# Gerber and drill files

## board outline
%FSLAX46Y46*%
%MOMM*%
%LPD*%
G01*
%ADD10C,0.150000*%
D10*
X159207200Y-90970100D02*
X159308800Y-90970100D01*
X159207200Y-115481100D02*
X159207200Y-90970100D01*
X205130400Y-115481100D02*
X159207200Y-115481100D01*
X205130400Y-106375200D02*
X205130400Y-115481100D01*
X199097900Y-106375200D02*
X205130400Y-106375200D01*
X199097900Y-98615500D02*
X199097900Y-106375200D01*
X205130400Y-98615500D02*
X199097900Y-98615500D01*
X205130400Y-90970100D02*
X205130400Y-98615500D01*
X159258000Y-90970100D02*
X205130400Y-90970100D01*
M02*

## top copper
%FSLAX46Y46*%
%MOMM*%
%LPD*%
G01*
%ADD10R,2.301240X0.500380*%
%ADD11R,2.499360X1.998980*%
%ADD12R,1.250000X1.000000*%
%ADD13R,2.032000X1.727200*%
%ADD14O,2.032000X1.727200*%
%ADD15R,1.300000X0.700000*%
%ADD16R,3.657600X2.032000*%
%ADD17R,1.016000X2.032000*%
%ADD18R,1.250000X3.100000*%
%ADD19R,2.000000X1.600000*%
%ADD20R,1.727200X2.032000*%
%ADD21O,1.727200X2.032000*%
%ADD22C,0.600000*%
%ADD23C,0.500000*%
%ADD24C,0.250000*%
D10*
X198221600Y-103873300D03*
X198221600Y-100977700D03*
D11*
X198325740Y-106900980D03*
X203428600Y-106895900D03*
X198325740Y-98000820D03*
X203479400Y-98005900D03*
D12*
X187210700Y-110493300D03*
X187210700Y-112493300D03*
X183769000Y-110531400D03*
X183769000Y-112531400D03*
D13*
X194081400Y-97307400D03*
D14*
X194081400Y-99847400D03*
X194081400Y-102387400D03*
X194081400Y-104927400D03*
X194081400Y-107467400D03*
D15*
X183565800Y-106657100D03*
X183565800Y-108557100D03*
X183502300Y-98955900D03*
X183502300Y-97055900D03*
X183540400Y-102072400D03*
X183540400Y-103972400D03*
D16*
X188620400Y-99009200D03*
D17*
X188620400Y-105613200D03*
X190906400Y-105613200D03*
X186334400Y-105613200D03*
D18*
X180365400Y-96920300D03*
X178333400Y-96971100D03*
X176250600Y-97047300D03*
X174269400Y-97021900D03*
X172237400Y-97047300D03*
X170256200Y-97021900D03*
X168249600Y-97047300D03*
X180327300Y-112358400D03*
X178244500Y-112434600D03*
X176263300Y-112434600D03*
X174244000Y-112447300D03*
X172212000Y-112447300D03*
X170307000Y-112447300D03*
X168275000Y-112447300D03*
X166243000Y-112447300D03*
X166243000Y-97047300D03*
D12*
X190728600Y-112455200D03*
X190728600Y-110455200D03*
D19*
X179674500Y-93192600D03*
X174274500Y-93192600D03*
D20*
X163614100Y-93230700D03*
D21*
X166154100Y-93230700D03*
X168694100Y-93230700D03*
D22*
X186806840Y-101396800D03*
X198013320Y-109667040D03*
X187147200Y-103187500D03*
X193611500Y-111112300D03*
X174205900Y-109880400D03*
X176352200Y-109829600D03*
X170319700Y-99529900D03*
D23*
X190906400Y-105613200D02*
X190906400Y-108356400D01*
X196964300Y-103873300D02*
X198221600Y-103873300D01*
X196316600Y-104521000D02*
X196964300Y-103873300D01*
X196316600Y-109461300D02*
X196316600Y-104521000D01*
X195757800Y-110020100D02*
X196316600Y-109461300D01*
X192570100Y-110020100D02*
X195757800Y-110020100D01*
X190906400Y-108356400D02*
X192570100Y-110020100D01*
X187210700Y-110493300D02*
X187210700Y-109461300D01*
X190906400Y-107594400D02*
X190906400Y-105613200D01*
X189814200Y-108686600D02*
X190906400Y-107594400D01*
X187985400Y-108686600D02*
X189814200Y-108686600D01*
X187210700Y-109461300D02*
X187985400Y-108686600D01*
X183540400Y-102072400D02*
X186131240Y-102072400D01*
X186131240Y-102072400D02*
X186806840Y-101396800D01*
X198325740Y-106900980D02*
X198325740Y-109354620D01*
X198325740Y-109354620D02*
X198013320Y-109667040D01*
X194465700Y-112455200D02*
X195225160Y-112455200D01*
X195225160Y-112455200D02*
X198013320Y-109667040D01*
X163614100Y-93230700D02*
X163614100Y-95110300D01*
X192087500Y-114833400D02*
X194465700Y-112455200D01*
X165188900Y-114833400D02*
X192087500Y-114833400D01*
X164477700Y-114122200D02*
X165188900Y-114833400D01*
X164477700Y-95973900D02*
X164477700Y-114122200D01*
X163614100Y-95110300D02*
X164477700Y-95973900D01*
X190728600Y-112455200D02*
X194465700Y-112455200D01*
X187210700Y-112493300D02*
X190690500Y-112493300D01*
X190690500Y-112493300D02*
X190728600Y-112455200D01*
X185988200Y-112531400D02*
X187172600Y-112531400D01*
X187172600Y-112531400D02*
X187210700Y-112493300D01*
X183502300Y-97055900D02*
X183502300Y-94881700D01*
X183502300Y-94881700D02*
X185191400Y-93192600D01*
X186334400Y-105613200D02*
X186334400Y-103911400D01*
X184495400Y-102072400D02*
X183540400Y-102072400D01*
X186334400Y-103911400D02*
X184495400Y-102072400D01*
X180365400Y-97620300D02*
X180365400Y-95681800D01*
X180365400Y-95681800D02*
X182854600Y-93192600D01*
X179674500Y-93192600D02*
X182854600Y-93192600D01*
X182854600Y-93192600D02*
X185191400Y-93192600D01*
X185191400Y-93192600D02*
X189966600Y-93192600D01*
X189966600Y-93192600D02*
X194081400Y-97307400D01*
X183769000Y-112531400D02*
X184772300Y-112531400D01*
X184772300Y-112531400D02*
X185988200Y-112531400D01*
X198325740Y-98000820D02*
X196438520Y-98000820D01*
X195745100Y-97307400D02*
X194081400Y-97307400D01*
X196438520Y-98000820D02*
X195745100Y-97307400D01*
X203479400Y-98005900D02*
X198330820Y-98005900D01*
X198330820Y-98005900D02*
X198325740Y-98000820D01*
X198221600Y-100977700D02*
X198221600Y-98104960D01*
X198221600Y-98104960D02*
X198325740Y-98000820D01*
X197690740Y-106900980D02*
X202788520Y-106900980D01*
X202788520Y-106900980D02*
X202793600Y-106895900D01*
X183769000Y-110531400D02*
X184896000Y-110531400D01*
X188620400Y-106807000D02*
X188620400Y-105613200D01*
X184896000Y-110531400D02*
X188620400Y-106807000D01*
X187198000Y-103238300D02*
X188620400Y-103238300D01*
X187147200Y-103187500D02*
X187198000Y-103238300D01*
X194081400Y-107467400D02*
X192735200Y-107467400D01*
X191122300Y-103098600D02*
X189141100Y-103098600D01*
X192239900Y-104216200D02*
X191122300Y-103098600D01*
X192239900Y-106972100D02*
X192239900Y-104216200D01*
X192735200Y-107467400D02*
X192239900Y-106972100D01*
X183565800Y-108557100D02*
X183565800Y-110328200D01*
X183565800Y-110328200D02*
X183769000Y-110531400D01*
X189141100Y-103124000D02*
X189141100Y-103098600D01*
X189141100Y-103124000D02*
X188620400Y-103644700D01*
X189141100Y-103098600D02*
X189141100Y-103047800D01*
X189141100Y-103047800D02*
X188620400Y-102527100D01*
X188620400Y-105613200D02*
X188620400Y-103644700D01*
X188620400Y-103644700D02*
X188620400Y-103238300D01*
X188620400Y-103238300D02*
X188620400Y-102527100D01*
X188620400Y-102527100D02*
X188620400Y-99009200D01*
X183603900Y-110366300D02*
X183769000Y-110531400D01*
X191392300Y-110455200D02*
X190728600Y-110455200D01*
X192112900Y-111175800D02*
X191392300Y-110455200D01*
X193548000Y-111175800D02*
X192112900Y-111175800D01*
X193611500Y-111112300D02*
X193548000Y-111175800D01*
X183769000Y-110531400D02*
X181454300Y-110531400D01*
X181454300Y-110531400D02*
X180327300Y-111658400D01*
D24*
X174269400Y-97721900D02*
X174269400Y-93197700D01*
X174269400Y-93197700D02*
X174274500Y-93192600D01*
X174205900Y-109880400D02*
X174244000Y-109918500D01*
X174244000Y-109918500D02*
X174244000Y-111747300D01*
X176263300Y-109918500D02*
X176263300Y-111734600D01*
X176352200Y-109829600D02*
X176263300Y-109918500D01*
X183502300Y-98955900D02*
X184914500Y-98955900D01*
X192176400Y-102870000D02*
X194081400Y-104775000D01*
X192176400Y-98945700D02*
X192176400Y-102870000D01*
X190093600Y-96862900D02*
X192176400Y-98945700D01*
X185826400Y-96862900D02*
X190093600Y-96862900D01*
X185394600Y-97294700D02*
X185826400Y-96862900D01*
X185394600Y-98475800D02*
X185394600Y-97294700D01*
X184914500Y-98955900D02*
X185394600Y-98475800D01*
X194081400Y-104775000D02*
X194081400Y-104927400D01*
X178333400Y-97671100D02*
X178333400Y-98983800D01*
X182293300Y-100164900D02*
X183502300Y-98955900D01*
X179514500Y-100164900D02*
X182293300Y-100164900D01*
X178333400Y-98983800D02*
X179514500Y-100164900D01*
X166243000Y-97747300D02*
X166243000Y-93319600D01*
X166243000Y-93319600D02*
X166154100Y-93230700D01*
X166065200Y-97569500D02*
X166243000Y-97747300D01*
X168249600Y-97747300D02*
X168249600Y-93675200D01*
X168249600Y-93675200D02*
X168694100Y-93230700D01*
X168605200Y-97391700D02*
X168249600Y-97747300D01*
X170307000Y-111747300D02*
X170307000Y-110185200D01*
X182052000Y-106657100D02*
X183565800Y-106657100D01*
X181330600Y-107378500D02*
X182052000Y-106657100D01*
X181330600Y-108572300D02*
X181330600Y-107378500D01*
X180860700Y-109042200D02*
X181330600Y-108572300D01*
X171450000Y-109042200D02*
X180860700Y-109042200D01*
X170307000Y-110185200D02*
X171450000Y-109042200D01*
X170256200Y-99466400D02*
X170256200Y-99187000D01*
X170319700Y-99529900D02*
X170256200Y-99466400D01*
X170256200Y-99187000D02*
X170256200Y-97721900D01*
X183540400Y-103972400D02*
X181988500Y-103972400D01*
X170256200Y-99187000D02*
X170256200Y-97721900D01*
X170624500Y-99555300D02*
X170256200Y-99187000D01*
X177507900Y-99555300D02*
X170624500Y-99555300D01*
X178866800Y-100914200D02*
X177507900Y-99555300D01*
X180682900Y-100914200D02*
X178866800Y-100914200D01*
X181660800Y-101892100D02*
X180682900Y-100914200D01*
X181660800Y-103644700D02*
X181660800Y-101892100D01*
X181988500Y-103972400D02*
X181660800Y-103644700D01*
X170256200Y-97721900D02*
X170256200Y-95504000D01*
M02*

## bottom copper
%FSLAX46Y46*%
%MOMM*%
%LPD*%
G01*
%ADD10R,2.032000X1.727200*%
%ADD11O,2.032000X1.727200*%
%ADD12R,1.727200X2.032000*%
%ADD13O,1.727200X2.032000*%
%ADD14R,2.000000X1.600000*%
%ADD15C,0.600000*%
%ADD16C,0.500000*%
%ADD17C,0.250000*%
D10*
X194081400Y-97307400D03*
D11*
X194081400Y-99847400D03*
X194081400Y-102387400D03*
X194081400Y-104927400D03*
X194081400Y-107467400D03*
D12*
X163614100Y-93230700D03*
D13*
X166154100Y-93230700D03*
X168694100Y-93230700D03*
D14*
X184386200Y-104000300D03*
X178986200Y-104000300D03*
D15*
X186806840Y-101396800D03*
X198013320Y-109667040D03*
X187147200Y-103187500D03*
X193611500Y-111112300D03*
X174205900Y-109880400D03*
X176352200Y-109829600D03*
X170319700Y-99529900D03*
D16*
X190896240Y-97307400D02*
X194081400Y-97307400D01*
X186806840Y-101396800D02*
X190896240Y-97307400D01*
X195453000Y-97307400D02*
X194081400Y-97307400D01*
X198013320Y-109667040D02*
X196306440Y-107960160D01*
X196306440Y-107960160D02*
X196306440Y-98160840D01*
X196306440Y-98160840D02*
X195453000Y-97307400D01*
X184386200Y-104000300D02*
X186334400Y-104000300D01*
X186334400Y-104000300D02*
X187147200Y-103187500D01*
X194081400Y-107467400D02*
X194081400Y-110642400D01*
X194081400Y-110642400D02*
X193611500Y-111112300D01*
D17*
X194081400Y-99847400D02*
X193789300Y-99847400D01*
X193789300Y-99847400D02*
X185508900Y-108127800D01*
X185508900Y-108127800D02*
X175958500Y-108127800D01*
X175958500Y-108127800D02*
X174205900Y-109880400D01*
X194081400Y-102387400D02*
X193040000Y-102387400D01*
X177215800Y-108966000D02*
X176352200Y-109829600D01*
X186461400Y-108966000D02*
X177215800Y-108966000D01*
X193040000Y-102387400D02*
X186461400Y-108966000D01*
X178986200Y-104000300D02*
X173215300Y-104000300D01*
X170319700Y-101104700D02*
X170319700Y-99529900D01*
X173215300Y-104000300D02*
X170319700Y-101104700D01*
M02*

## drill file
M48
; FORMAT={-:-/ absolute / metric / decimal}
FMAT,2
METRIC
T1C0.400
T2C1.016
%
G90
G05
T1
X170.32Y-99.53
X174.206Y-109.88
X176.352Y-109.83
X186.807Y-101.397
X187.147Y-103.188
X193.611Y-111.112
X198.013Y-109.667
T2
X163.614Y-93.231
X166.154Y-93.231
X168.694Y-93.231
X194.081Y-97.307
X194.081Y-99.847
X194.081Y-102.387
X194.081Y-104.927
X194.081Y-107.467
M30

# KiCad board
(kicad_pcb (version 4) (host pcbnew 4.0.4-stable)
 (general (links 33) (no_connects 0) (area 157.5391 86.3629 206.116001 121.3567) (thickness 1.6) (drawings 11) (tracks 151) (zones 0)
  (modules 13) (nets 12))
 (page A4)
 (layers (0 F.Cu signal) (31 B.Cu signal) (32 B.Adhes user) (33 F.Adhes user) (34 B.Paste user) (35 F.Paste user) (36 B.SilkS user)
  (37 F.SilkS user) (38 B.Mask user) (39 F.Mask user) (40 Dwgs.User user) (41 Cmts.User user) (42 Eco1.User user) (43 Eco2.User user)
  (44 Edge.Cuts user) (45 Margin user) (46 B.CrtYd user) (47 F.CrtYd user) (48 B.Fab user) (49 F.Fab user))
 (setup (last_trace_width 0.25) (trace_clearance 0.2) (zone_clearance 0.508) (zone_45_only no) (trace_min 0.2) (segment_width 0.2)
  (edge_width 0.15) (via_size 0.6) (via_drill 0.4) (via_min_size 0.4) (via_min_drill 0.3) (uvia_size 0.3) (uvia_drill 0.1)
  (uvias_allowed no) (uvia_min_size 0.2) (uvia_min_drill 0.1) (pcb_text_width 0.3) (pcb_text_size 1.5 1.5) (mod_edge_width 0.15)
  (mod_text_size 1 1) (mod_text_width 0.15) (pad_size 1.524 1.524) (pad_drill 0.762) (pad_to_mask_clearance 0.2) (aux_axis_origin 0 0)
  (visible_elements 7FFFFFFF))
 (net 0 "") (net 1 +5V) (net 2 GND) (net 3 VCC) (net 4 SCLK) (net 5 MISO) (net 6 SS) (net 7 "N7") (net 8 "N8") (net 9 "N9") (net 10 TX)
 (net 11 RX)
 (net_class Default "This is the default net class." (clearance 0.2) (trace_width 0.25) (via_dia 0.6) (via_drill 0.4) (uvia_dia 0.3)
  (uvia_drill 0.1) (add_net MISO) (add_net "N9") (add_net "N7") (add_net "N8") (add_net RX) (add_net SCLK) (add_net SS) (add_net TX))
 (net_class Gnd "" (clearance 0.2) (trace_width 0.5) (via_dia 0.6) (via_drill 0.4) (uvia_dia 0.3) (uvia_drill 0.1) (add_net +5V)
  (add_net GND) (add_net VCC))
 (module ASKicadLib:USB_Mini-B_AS (layer F.Cu) (at 201.676 102.4509 180)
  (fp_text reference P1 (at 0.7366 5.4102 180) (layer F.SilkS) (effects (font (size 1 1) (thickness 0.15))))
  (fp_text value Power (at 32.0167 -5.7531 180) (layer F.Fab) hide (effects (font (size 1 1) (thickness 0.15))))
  (pad 1 smd rect (at 3.4544 -1.4224 180) (size 2.30124 0.50038) (layers F.Cu F.Paste F.Mask) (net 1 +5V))
  (pad 5 smd rect (at 3.4544 1.4732 180) (size 2.30124 0.50038) (layers F.Cu F.Paste F.Mask) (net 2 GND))
  (pad 6 smd rect (at 3.35026 -4.45008 180) (size 2.49936 1.99898) (layers F.Cu F.Paste F.Mask) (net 2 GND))
  (pad 6 smd rect (at -1.7526 -4.445 180) (size 2.49936 1.99898) (layers F.Cu F.Paste F.Mask) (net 2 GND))
  (pad 6 smd rect (at 3.35026 4.45008 180) (size 2.49936 1.99898) (layers F.Cu F.Paste F.Mask) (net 2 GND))
  (pad 6 smd rect (at -1.8034 4.445 180) (size 2.49936 1.99898) (layers F.Cu F.Paste F.Mask) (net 2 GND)))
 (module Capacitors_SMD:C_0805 (layer F.Cu) (at 187.2107 111.4933 270)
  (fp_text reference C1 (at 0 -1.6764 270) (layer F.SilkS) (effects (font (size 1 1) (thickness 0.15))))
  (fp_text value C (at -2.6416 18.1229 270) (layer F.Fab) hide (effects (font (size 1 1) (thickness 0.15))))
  (pad 1 smd rect (at -1 0 270) (size 1 1.25) (layers F.Cu F.Paste F.Mask) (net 1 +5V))
  (pad 2 smd rect (at 1 0 270) (size 1 1.25) (layers F.Cu F.Paste F.Mask) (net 2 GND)))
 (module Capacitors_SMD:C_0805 (layer F.Cu) (at 183.769 111.5314 270)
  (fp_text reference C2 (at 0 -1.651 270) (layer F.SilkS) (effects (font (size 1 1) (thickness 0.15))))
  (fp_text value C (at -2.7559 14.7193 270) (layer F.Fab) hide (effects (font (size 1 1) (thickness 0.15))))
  (pad 1 smd rect (at -1 0 270) (size 1 1.25) (layers F.Cu F.Paste F.Mask) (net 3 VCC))
  (pad 2 smd rect (at 1 0 270) (size 1 1.25) (layers F.Cu F.Paste F.Mask) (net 2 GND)))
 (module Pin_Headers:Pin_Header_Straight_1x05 (layer F.Cu) (at 194.0814 97.3074)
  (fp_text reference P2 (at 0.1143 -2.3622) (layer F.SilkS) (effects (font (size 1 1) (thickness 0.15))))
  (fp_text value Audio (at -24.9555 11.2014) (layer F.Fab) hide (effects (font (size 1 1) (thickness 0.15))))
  (pad 1 thru_hole rect (at 0 0) (size 2.032 1.7272) (drill 1.016) (layers *.Cu *.Mask) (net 2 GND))
  (pad 2 thru_hole oval (at 0 2.54) (size 2.032 1.7272) (drill 1.016) (layers *.Cu *.Mask) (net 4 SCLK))
  (pad 3 thru_hole oval (at 0 5.08) (size 2.032 1.7272) (drill 1.016) (layers *.Cu *.Mask) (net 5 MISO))
  (pad 4 thru_hole oval (at 0 7.62) (size 2.032 1.7272) (drill 1.016) (layers *.Cu *.Mask) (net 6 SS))
  (pad 5 thru_hole oval (at 0 10.16) (size 2.032 1.7272) (drill 1.016) (layers *.Cu *.Mask) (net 3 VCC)))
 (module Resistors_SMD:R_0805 (layer F.Cu) (at 183.5658 107.6071 270)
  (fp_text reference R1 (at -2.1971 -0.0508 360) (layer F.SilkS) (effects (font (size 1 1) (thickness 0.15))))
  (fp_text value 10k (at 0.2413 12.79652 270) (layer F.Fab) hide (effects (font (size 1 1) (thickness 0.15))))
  (pad 1 smd rect (at -0.95 0 270) (size 0.7 1.3) (layers F.Cu F.Paste F.Mask) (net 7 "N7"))
  (pad 2 smd rect (at 0.95 0 270) (size 0.7 1.3) (layers F.Cu F.Paste F.Mask) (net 3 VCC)))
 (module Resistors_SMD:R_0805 (layer F.Cu) (at 183.5023 98.0059 90)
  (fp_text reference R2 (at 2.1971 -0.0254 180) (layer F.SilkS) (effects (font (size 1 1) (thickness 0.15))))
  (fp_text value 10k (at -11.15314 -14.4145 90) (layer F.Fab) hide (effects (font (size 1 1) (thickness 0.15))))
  (pad 1 smd rect (at -0.95 0 90) (size 0.7 1.3) (layers F.Cu F.Paste F.Mask) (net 6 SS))
  (pad 2 smd rect (at 0.95 0 90) (size 0.7 1.3) (layers F.Cu F.Paste F.Mask) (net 2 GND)))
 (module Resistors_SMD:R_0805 (layer F.Cu) (at 183.5404 103.0224 270)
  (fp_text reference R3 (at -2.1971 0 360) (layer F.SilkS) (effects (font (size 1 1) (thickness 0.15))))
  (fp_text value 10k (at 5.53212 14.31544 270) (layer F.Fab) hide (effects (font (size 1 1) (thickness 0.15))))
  (pad 1 smd rect (at -0.95 0 270) (size 0.7 1.3) (layers F.Cu F.Paste F.Mask) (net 2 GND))
  (pad 2 smd rect (at 0.95 0 270) (size 0.7 1.3) (layers F.Cu F.Paste F.Mask) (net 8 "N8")))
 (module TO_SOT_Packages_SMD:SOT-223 (layer F.Cu) (at 188.6204 102.3112)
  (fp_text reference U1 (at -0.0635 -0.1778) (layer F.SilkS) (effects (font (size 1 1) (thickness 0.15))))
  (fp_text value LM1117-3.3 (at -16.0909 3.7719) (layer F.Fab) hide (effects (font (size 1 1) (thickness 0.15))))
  (pad 4 smd rect (at 0 -3.302) (size 3.6576 2.032) (layers F.Cu F.Paste F.Mask) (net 3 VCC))
  (pad 2 smd rect (at 0 3.302) (size 1.016 2.032) (layers F.Cu F.Paste F.Mask) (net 3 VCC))
  (pad 3 smd rect (at 2.286 3.302) (size 1.016 2.032) (layers F.Cu F.Paste F.Mask) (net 1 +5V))
  (pad 1 smd rect (at -2.286 3.302) (size 1.016 2.032) (layers F.Cu F.Paste F.Mask) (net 2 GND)))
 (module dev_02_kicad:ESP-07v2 (layer F.Cu) (at 166.243 111.7473 90)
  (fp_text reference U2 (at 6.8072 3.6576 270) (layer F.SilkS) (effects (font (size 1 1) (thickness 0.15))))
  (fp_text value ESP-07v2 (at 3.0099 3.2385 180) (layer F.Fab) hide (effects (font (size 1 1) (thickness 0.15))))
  (pad 9 smd rect (at 14.127 14.1224 90) (size 3.1 1.25) (drill (offset 0.7 0)) (layers F.Cu F.Paste F.Mask) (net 2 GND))
  (pad 10 smd rect (at 14.0762 12.0904 90) (size 3.1 1.25) (drill (offset 0.7 0)) (layers F.Cu F.Paste F.Mask) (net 6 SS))
  (pad 11 smd rect (at 14 10.0076 90) (size 3.1 1.25) (drill (offset 0.7 0)) (layers F.Cu F.Paste F.Mask))
  (pad 12 smd rect (at 14.0254 8.0264 90) (size 3.1 1.25) (drill (offset 0.7 0)) (layers F.Cu F.Paste F.Mask) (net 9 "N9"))
  (pad 13 smd rect (at 14 5.9944 90) (size 3.1 1.25) (drill (offset 0.7 0)) (layers F.Cu F.Paste F.Mask))
  (pad 14 smd rect (at 14.0254 4.0132 90) (size 3.1 1.25) (drill (offset 0.7 0)) (layers F.Cu F.Paste F.Mask) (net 8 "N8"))
  (pad 15 smd rect (at 14 2.0066 90) (size 3.1 1.25) (drill (offset 0.7 0)) (layers F.Cu F.Paste F.Mask) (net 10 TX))
  (pad 8 smd rect (at 0.0889 14.0843 90) (size 3.1 1.25) (drill (offset -0.7 0)) (layers F.Cu F.Paste F.Mask) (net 3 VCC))
  (pad 7 smd rect (at 0.0127 12.0015 90) (size 3.1 1.25) (drill (offset -0.7 0)) (layers F.Cu F.Paste F.Mask))
  (pad 6 smd rect (at 0.0127 10.0203 90) (size 3.1 1.25) (drill (offset -0.7 0)) (layers F.Cu F.Paste F.Mask) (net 5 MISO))
  (pad 5 smd rect (at 0 8.001 90) (size 3.1 1.25) (drill (offset -0.7 0)) (layers F.Cu F.Paste F.Mask) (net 4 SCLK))
  (pad 4 smd rect (at 0 5.969 90) (size 3.1 1.25) (drill (offset -0.7 0)) (layers F.Cu F.Paste F.Mask))
  (pad 3 smd rect (at 0 4.064 90) (size 3.1 1.25) (drill (offset -0.7 0)) (layers F.Cu F.Paste F.Mask) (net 7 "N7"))
  (pad 2 smd rect (at 0 2.032 90) (size 3.1 1.25) (drill (offset -0.7 0)) (layers F.Cu F.Paste F.Mask))
  (pad 1 smd rect (at 0 0 90) (size 3.1 1.25) (drill (offset -0.7 0)) (layers F.Cu F.Paste F.Mask))
  (pad 16 smd rect (at 14 0 90) (size 3.1 1.25) (drill (offset 0.7 0)) (layers F.Cu F.Paste F.Mask) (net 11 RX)))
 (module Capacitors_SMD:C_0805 (layer F.Cu) (at 190.7286 111.4552 90)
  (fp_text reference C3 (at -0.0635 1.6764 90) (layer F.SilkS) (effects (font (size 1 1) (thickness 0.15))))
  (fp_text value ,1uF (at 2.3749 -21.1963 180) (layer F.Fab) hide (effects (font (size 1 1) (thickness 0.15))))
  (pad 1 smd rect (at -1 0 90) (size 1 1.25) (layers F.Cu F.Paste F.Mask) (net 2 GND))
  (pad 2 smd rect (at 1 0 90) (size 1 1.25) (layers F.Cu F.Paste F.Mask) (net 3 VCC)))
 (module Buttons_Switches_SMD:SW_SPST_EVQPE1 (layer F.Cu) (at 176.9745 93.1926)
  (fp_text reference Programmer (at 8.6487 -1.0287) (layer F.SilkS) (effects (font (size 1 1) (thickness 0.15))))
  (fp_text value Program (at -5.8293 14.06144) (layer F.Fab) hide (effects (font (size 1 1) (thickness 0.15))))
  (pad 2 smd rect (at 2.7 0) (size 2 1.6) (layers F.Cu F.Paste F.Mask) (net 2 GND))
  (pad 1 smd rect (at -2.7 0) (size 2 1.6) (layers F.Cu F.Paste F.Mask) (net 9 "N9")))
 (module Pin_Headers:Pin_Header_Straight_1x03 (layer F.Cu) (at 163.6141 93.2307 90)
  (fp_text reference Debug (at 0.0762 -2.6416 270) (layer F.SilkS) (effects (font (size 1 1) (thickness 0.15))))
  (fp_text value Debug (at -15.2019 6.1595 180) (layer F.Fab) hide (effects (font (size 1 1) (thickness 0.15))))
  (pad 1 thru_hole rect (at 0 0 90) (size 2.032 1.7272) (drill 1.016) (layers *.Cu *.Mask) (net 2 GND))
  (pad 2 thru_hole oval (at 0 2.54 90) (size 2.032 1.7272) (drill 1.016) (layers *.Cu *.Mask) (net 11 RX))
  (pad 3 thru_hole oval (at 0 5.08 90) (size 2.032 1.7272) (drill 1.016) (layers *.Cu *.Mask) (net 10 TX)))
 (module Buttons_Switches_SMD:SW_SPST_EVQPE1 (layer B.Cu) (at 181.6862 104.0003)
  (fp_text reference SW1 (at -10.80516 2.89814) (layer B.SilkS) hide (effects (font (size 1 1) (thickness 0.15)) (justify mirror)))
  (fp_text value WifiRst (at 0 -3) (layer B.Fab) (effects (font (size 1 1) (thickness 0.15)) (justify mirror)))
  (pad 2 smd rect (at 2.7 0) (size 2 1.6) (layers B.Cu B.Paste B.Mask) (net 3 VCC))
  (pad 1 smd rect (at -2.7 0) (size 2 1.6) (layers B.Cu B.Paste B.Mask) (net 8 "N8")))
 (gr_line (start 159.2072 90.9701) (end 159.3088 90.9701) (angle 90) (layer Edge.Cuts) (width 0.15))
 (gr_line (start 159.2072 115.4811) (end 159.2072 90.9701) (angle 90) (layer Edge.Cuts) (width 0.15))
 (gr_line (start 205.1304 115.4811) (end 159.2072 115.4811) (angle 90) (layer Edge.Cuts) (width 0.15))
 (gr_line (start 205.1304 106.3752) (end 205.1304 115.4811) (angle 90) (layer Edge.Cuts) (width 0.15))
 (gr_line (start 199.0979 106.3752) (end 205.1304 106.3752) (angle 90) (layer Edge.Cuts) (width 0.15))
 (gr_line (start 199.0979 98.6155) (end 199.0979 106.3752) (angle 90) (layer Edge.Cuts) (width 0.15))
 (gr_line (start 205.1304 98.6155) (end 199.0979 98.6155) (angle 90) (layer Edge.Cuts) (width 0.15))
 (gr_line (start 205.1304 90.9701) (end 205.1304 98.6155) (angle 90) (layer Edge.Cuts) (width 0.15))
 (gr_line (start 159.258 90.9701) (end 205.1304 90.9701) (angle 90) (layer Edge.Cuts) (width 0.15))
 (segment (start 190.9064 105.6132) (end 190.9064 108.3564) (width 0.5) (layer F.Cu) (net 1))
 (segment (start 196.9643 103.8733) (end 198.2216 103.8733) (width 0.5) (layer F.Cu) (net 1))
 (segment (start 196.3166 104.521) (end 196.9643 103.8733) (width 0.5) (layer F.Cu) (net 1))
 (segment (start 196.3166 109.4613) (end 196.3166 104.521) (width 0.5) (layer F.Cu) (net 1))
 (segment (start 195.7578 110.0201) (end 196.3166 109.4613) (width 0.5) (layer F.Cu) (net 1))
 (segment (start 192.5701 110.0201) (end 195.7578 110.0201) (width 0.5) (layer F.Cu) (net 1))
 (segment (start 190.9064 108.3564) (end 192.5701 110.0201) (width 0.5) (layer F.Cu) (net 1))
 (segment (start 187.2107 110.4933) (end 187.2107 109.4613) (width 0.5) (layer F.Cu) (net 1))
 (segment (start 190.9064 107.5944) (end 190.9064 105.6132) (width 0.5) (layer F.Cu) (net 1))
 (segment (start 189.8142 108.6866) (end 190.9064 107.5944) (width 0.5) (layer F.Cu) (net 1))
 (segment (start 187.9854 108.6866) (end 189.8142 108.6866) (width 0.5) (layer F.Cu) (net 1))
 (segment (start 187.2107 109.4613) (end 187.9854 108.6866) (width 0.5) (layer F.Cu) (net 1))
 (segment (start 183.5404 102.0724) (end 186.13124 102.0724) (width 0.5) (layer F.Cu) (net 2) (status 400000))
 (segment (start 190.89624 97.3074) (end 194.0814 97.3074) (width 0.5) (layer B.Cu) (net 2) (status 800000))
 (segment (start 186.80684 101.3968) (end 190.89624 97.3074) (width 0.5) (layer B.Cu) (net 2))
 (via (at 186.80684 101.3968) (size 0.6) (drill 0.4) (layers F.Cu B.Cu) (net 2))
 (segment (start 186.13124 102.0724) (end 186.80684 101.3968) (width 0.5) (layer F.Cu) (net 2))
 (segment (start 198.32574 106.90098) (end 198.32574 109.35462) (width 0.5) (layer F.Cu) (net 2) (status 400000))
 (segment (start 198.32574 109.35462) (end 198.01332 109.66704) (width 0.5) (layer F.Cu) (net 2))
 (segment (start 194.4657 112.4552) (end 195.22516 112.4552) (width 0.5) (layer F.Cu) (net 2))
 (segment (start 195.453 97.3074) (end 194.0814 97.3074) (width 0.5) (layer B.Cu) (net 2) (status 800000))
 (via (at 198.01332 109.66704) (size 0.6) (drill 0.4) (layers F.Cu B.Cu) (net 2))
 (segment (start 198.01332 109.66704) (end 196.30644 107.96016) (width 0.5) (layer B.Cu) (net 2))
 (segment (start 196.30644 107.96016) (end 196.30644 98.16084) (width 0.5) (layer B.Cu) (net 2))
 (segment (start 196.30644 98.16084) (end 195.453 97.3074) (width 0.5) (layer B.Cu) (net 2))
 (segment (start 195.22516 112.4552) (end 198.01332 109.66704) (width 0.5) (layer F.Cu) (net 2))
 (segment (start 163.6141 93.2307) (end 163.6141 95.1103) (width 0.5) (layer F.Cu) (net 2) (status 400000))
 (segment (start 192.0875 114.8334) (end 194.4657 112.4552) (width 0.5) (layer F.Cu) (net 2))
 (segment (start 165.1889 114.8334) (end 192.0875 114.8334) (width 0.5) (layer F.Cu) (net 2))
 (segment (start 164.4777 114.1222) (end 165.1889 114.8334) (width 0.5) (layer F.Cu) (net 2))
 (segment (start 164.4777 95.9739) (end 164.4777 114.1222) (width 0.5) (layer F.Cu) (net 2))
 (segment (start 163.6141 95.1103) (end 164.4777 95.9739) (width 0.5) (layer F.Cu) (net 2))
 (segment (start 190.7286 112.4552) (end 194.4657 112.4552) (width 0.5) (layer F.Cu) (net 2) (status 400000))
 (segment (start 187.2107 112.4933) (end 190.6905 112.4933) (width 0.5) (layer F.Cu) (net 2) (status C00000))
 (segment (start 190.6905 112.4933) (end 190.7286 112.4552) (width 0.5) (layer F.Cu) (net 2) (status C00000))
 (segment (start 185.9882 112.5314) (end 187.1726 112.5314) (width 0.5) (layer F.Cu) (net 2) (status 800000))
 (segment (start 187.1726 112.5314) (end 187.2107 112.4933) (width 0.5) (layer F.Cu) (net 2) (status C00000))
 (segment (start 183.5023 97.0559) (end 183.5023 94.8817) (width 0.5) (layer F.Cu) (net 2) (status 400000))
 (segment (start 183.5023 94.8817) (end 185.1914 93.1926) (width 0.5) (layer F.Cu) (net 2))
 (segment (start 186.3344 105.6132) (end 186.3344 103.9114) (width 0.5) (layer F.Cu) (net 2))
 (segment (start 184.4954 102.0724) (end 183.5404 102.0724) (width 0.5) (layer F.Cu) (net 2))
 (segment (start 186.3344 103.9114) (end 184.4954 102.0724) (width 0.5) (layer F.Cu) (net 2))
 (segment (start 180.3654 97.6203) (end 180.3654 95.6818) (width 0.5) (layer F.Cu) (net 2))
 (segment (start 180.3654 95.6818) (end 182.8546 93.1926) (width 0.5) (layer F.Cu) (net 2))
 (segment (start 179.6745 93.1926) (end 182.8546 93.1926) (width 0.5) (layer F.Cu) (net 2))
 (segment (start 182.8546 93.1926) (end 185.1914 93.1926) (width 0.5) (layer F.Cu) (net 2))
 (segment (start 185.1914 93.1926) (end 189.9666 93.1926) (width 0.5) (layer F.Cu) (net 2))
 (segment (start 189.9666 93.1926) (end 194.0814 97.3074) (width 0.5) (layer F.Cu) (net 2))
 (segment (start 183.769 112.5314) (end 184.7723 112.5314) (width 0.5) (layer F.Cu) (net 2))
 (segment (start 184.7723 112.5314) (end 185.9882 112.5314) (width 0.5) (layer F.Cu) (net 2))
 (segment (start 198.32574 98.00082) (end 196.43852 98.00082) (width 0.5) (layer F.Cu) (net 2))
 (segment (start 195.7451 97.3074) (end 194.0814 97.3074) (width 0.5) (layer F.Cu) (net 2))
 (segment (start 196.43852 98.00082) (end 195.7451 97.3074) (width 0.5) (layer F.Cu) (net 2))
 (segment (start 203.4794 98.0059) (end 198.33082 98.0059) (width 0.5) (layer F.Cu) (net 2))
 (segment (start 198.33082 98.0059) (end 198.32574 98.00082) (width 0.5) (layer F.Cu) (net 2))
 (segment (start 198.2216 100.9777) (end 198.2216 98.10496) (width 0.5) (layer F.Cu) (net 2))
 (segment (start 198.2216 98.10496) (end 198.32574 98.00082) (width 0.5) (layer F.Cu) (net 2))
 (segment (start 197.69074 106.90098) (end 202.78852 106.90098) (width 0.5) (layer F.Cu) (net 2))
 (segment (start 202.78852 106.90098) (end 202.7936 106.8959) (width 0.5) (layer F.Cu) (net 2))
 (segment (start 183.769 110.5314) (end 184.896 110.5314) (width 0.5) (layer F.Cu) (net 3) (status 400000))
 (segment (start 188.6204 106.807) (end 188.6204 105.6132) (width 0.5) (layer F.Cu) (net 3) (status 800000))
 (segment (start 184.896 110.5314) (end 188.6204 106.807) (width 0.5) (layer F.Cu) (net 3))
 (segment (start 184.3862 104.0003) (end 186.3344 104.0003) (width 0.5) (layer B.Cu) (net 3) (status 400000))
 (segment (start 187.198 103.2383) (end 188.6204 103.2383) (width 0.5) (layer F.Cu) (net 3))
 (segment (start 187.1472 103.1875) (end 187.198 103.2383) (width 0.5) (layer F.Cu) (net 3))
 (via (at 187.1472 103.1875) (size 0.6) (drill 0.4) (layers F.Cu B.Cu) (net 3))
 (segment (start 186.3344 104.0003) (end 187.1472 103.1875) (width 0.5) (layer B.Cu) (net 3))
 (segment (start 194.0814 107.4674) (end 192.7352 107.4674) (width 0.5) (layer F.Cu) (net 3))
 (segment (start 191.1223 103.0986) (end 189.1411 103.0986) (width 0.5) (layer F.Cu) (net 3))
 (segment (start 192.2399 104.2162) (end 191.1223 103.0986) (width 0.5) (layer F.Cu) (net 3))
 (segment (start 192.2399 106.9721) (end 192.2399 104.2162) (width 0.5) (layer F.Cu) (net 3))
 (segment (start 192.7352 107.4674) (end 192.2399 106.9721) (width 0.5) (layer F.Cu) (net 3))
 (segment (start 183.5658 108.5571) (end 183.5658 110.3282) (width 0.5) (layer F.Cu) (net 3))
 (segment (start 183.5658 110.3282) (end 183.769 110.5314) (width 0.5) (layer F.Cu) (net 3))
 (segment (start 189.1411 103.124) (end 189.1411 103.0986) (width 0.5) (layer F.Cu) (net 3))
 (segment (start 189.1411 103.124) (end 188.6204 103.6447) (width 0.5) (layer F.Cu) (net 3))
 (segment (start 189.1411 103.0986) (end 189.1411 103.0478) (width 0.5) (layer F.Cu) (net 3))
 (segment (start 189.1411 103.0478) (end 188.6204 102.5271) (width 0.5) (layer F.Cu) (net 3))
 (segment (start 188.6204 105.6132) (end 188.6204 103.6447) (width 0.5) (layer F.Cu) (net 3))
 (segment (start 188.6204 103.6447) (end 188.6204 103.2383) (width 0.5) (layer F.Cu) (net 3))
 (segment (start 188.6204 103.2383) (end 188.6204 102.5271) (width 0.5) (layer F.Cu) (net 3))
 (segment (start 188.6204 102.5271) (end 188.6204 99.0092) (width 0.5) (layer F.Cu) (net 3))
 (segment (start 183.6039 110.3663) (end 183.769 110.5314) (width 0.5) (layer F.Cu) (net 3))
 (segment (start 194.0814 107.4674) (end 194.0814 110.6424) (width 0.5) (layer B.Cu) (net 3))
 (segment (start 191.3923 110.4552) (end 190.7286 110.4552) (width 0.5) (layer F.Cu) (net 3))
 (segment (start 192.1129 111.1758) (end 191.3923 110.4552) (width 0.5) (layer F.Cu) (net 3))
 (segment (start 193.548 111.1758) (end 192.1129 111.1758) (width 0.5) (layer F.Cu) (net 3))
 (segment (start 193.6115 111.1123) (end 193.548 111.1758) (width 0.5) (layer F.Cu) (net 3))
 (via (at 193.6115 111.1123) (size 0.6) (drill 0.4) (layers F.Cu B.Cu) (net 3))
 (segment (start 194.0814 110.6424) (end 193.6115 111.1123) (width 0.5) (layer B.Cu) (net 3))
 (segment (start 183.769 110.5314) (end 181.4543 110.5314) (width 0.5) (layer F.Cu) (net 3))
 (segment (start 181.4543 110.5314) (end 180.3273 111.6584) (width 0.5) (layer F.Cu) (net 3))
 (segment (start 174.2694 97.7219) (end 174.2694 93.1977) (width 0.25) (layer F.Cu) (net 9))
 (segment (start 174.2694 93.1977) (end 174.2745 93.1926) (width 0.25) (layer F.Cu) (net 9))
 (segment (start 194.0814 99.8474) (end 193.7893 99.8474) (width 0.25) (layer B.Cu) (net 4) (status C00000))
 (segment (start 193.7893 99.8474) (end 185.5089 108.1278) (width 0.25) (layer B.Cu) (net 4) (status 400000))
 (segment (start 185.5089 108.1278) (end 175.9585 108.1278) (width 0.25) (layer B.Cu) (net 4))
 (segment (start 175.9585 108.1278) (end 174.2059 109.8804) (width 0.25) (layer B.Cu) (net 4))
 (via (at 174.2059 109.8804) (size 0.6) (drill 0.4) (layers F.Cu B.Cu) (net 4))
 (segment (start 174.2059 109.8804) (end 174.244 109.9185) (width 0.25) (layer F.Cu) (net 4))
 (segment (start 174.244 109.9185) (end 174.244 111.7473) (width 0.25) (layer F.Cu) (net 4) (status 800000))
 (segment (start 194.0814 102.3874) (end 193.04 102.3874) (width 0.25) (layer B.Cu) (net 5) (status 400000))
 (segment (start 176.2633 109.9185) (end 176.2633 111.7346) (width 0.25) (layer F.Cu) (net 5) (status 800000))
 (segment (start 176.3522 109.8296) (end 176.2633 109.9185) (width 0.25) (layer F.Cu) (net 5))
 (via (at 176.3522 109.8296) (size 0.6) (drill 0.4) (layers F.Cu B.Cu) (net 5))
 (segment (start 177.2158 108.966) (end 176.3522 109.8296) (width 0.25) (layer B.Cu) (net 5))
 (segment (start 186.4614 108.966) (end 177.2158 108.966) (width 0.25) (layer B.Cu) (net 5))
 (segment (start 193.04 102.3874) (end 186.4614 108.966) (width 0.25) (layer B.Cu) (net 5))
 (segment (start 183.5023 98.9559) (end 184.9145 98.9559) (width 0.25) (layer F.Cu) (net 6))
 (segment (start 192.1764 102.87) (end 194.0814 104.775) (width 0.25) (layer F.Cu) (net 6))
 (segment (start 192.1764 98.9457) (end 192.1764 102.87) (width 0.25) (layer F.Cu) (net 6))
 (segment (start 190.0936 96.8629) (end 192.1764 98.9457) (width 0.25) (layer F.Cu) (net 6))
 (segment (start 185.8264 96.8629) (end 190.0936 96.8629) (width 0.25) (layer F.Cu) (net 6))
 (segment (start 185.3946 97.2947) (end 185.8264 96.8629) (width 0.25) (layer F.Cu) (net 6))
 (segment (start 185.3946 98.4758) (end 185.3946 97.2947) (width 0.25) (layer F.Cu) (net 6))
 (segment (start 184.9145 98.9559) (end 185.3946 98.4758) (width 0.25) (layer F.Cu) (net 6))
 (segment (start 194.0814 104.775) (end 194.0814 104.9274) (width 0.25) (layer F.Cu) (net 6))
 (segment (start 178.3334 97.6711) (end 178.3334 98.9838) (width 0.25) (layer F.Cu) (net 6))
 (segment (start 182.2933 100.1649) (end 183.5023 98.9559) (width 0.25) (layer F.Cu) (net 6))
 (segment (start 179.5145 100.1649) (end 182.2933 100.1649) (width 0.25) (layer F.Cu) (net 6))
 (segment (start 178.3334 98.9838) (end 179.5145 100.1649) (width 0.25) (layer F.Cu) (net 6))
 (segment (start 166.243 97.7473) (end 166.243 93.3196) (width 0.25) (layer F.Cu) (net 11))
 (segment (start 166.243 93.3196) (end 166.1541 93.2307) (width 0.25) (layer F.Cu) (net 11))
 (segment (start 166.0652 97.5695) (end 166.243 97.7473) (width 0.25) (layer F.Cu) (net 11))
 (segment (start 168.2496 97.7473) (end 168.2496 93.6752) (width 0.25) (layer F.Cu) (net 10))
 (segment (start 168.2496 93.6752) (end 168.6941 93.2307) (width 0.25) (layer F.Cu) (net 10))
 (segment (start 168.6052 97.3917) (end 168.2496 97.7473) (width 0.25) (layer F.Cu) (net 10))
 (segment (start 170.307 111.7473) (end 170.307 110.1852) (width 0.25) (layer F.Cu) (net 7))
 (segment (start 182.052 106.6571) (end 183.5658 106.6571) (width 0.25) (layer F.Cu) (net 7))
 (segment (start 181.3306 107.3785) (end 182.052 106.6571) (width 0.25) (layer F.Cu) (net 7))
 (segment (start 181.3306 108.5723) (end 181.3306 107.3785) (width 0.25) (layer F.Cu) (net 7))
 (segment (start 180.8607 109.0422) (end 181.3306 108.5723) (width 0.25) (layer F.Cu) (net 7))
 (segment (start 171.45 109.0422) (end 180.8607 109.0422) (width 0.25) (layer F.Cu) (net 7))
 (segment (start 170.307 110.1852) (end 171.45 109.0422) (width 0.25) (layer F.Cu) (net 7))
 (segment (start 178.9862 104.0003) (end 173.2153 104.0003) (width 0.25) (layer B.Cu) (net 8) (status 400000))
 (segment (start 170.2562 99.4664) (end 170.2562 99.187) (width 0.25) (layer F.Cu) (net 8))
 (segment (start 170.3197 99.5299) (end 170.2562 99.4664) (width 0.25) (layer F.Cu) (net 8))
 (via (at 170.3197 99.5299) (size 0.6) (drill 0.4) (layers F.Cu B.Cu) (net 8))
 (segment (start 170.3197 101.1047) (end 170.3197 99.5299) (width 0.25) (layer B.Cu) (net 8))
 (segment (start 173.2153 104.0003) (end 170.3197 101.1047) (width 0.25) (layer B.Cu) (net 8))
 (segment (start 170.2562 99.187) (end 170.2562 97.7219) (width 0.25) (layer F.Cu) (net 8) (status 800000))
 (segment (start 183.5404 103.9724) (end 181.9885 103.9724) (width 0.25) (layer F.Cu) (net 8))
 (segment (start 170.2562 99.187) (end 170.2562 97.7219) (width 0.25) (layer F.Cu) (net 8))
 (segment (start 170.6245 99.5553) (end 170.2562 99.187) (width 0.25) (layer F.Cu) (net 8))
 (segment (start 177.5079 99.5553) (end 170.6245 99.5553) (width 0.25) (layer F.Cu) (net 8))
 (segment (start 178.8668 100.9142) (end 177.5079 99.5553) (width 0.25) (layer F.Cu) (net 8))
 (segment (start 180.6829 100.9142) (end 178.8668 100.9142) (width 0.25) (layer F.Cu) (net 8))
 (segment (start 181.6608 101.8921) (end 180.6829 100.9142) (width 0.25) (layer F.Cu) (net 8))
 (segment (start 181.6608 103.6447) (end 181.6608 101.8921) (width 0.25) (layer F.Cu) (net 8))
 (segment (start 181.9885 103.9724) (end 181.6608 103.6447) (width 0.25) (layer F.Cu) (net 8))
 (segment (start 170.2562 97.7219) (end 170.2562 95.504) (width 0.25) (layer F.Cu) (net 8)))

